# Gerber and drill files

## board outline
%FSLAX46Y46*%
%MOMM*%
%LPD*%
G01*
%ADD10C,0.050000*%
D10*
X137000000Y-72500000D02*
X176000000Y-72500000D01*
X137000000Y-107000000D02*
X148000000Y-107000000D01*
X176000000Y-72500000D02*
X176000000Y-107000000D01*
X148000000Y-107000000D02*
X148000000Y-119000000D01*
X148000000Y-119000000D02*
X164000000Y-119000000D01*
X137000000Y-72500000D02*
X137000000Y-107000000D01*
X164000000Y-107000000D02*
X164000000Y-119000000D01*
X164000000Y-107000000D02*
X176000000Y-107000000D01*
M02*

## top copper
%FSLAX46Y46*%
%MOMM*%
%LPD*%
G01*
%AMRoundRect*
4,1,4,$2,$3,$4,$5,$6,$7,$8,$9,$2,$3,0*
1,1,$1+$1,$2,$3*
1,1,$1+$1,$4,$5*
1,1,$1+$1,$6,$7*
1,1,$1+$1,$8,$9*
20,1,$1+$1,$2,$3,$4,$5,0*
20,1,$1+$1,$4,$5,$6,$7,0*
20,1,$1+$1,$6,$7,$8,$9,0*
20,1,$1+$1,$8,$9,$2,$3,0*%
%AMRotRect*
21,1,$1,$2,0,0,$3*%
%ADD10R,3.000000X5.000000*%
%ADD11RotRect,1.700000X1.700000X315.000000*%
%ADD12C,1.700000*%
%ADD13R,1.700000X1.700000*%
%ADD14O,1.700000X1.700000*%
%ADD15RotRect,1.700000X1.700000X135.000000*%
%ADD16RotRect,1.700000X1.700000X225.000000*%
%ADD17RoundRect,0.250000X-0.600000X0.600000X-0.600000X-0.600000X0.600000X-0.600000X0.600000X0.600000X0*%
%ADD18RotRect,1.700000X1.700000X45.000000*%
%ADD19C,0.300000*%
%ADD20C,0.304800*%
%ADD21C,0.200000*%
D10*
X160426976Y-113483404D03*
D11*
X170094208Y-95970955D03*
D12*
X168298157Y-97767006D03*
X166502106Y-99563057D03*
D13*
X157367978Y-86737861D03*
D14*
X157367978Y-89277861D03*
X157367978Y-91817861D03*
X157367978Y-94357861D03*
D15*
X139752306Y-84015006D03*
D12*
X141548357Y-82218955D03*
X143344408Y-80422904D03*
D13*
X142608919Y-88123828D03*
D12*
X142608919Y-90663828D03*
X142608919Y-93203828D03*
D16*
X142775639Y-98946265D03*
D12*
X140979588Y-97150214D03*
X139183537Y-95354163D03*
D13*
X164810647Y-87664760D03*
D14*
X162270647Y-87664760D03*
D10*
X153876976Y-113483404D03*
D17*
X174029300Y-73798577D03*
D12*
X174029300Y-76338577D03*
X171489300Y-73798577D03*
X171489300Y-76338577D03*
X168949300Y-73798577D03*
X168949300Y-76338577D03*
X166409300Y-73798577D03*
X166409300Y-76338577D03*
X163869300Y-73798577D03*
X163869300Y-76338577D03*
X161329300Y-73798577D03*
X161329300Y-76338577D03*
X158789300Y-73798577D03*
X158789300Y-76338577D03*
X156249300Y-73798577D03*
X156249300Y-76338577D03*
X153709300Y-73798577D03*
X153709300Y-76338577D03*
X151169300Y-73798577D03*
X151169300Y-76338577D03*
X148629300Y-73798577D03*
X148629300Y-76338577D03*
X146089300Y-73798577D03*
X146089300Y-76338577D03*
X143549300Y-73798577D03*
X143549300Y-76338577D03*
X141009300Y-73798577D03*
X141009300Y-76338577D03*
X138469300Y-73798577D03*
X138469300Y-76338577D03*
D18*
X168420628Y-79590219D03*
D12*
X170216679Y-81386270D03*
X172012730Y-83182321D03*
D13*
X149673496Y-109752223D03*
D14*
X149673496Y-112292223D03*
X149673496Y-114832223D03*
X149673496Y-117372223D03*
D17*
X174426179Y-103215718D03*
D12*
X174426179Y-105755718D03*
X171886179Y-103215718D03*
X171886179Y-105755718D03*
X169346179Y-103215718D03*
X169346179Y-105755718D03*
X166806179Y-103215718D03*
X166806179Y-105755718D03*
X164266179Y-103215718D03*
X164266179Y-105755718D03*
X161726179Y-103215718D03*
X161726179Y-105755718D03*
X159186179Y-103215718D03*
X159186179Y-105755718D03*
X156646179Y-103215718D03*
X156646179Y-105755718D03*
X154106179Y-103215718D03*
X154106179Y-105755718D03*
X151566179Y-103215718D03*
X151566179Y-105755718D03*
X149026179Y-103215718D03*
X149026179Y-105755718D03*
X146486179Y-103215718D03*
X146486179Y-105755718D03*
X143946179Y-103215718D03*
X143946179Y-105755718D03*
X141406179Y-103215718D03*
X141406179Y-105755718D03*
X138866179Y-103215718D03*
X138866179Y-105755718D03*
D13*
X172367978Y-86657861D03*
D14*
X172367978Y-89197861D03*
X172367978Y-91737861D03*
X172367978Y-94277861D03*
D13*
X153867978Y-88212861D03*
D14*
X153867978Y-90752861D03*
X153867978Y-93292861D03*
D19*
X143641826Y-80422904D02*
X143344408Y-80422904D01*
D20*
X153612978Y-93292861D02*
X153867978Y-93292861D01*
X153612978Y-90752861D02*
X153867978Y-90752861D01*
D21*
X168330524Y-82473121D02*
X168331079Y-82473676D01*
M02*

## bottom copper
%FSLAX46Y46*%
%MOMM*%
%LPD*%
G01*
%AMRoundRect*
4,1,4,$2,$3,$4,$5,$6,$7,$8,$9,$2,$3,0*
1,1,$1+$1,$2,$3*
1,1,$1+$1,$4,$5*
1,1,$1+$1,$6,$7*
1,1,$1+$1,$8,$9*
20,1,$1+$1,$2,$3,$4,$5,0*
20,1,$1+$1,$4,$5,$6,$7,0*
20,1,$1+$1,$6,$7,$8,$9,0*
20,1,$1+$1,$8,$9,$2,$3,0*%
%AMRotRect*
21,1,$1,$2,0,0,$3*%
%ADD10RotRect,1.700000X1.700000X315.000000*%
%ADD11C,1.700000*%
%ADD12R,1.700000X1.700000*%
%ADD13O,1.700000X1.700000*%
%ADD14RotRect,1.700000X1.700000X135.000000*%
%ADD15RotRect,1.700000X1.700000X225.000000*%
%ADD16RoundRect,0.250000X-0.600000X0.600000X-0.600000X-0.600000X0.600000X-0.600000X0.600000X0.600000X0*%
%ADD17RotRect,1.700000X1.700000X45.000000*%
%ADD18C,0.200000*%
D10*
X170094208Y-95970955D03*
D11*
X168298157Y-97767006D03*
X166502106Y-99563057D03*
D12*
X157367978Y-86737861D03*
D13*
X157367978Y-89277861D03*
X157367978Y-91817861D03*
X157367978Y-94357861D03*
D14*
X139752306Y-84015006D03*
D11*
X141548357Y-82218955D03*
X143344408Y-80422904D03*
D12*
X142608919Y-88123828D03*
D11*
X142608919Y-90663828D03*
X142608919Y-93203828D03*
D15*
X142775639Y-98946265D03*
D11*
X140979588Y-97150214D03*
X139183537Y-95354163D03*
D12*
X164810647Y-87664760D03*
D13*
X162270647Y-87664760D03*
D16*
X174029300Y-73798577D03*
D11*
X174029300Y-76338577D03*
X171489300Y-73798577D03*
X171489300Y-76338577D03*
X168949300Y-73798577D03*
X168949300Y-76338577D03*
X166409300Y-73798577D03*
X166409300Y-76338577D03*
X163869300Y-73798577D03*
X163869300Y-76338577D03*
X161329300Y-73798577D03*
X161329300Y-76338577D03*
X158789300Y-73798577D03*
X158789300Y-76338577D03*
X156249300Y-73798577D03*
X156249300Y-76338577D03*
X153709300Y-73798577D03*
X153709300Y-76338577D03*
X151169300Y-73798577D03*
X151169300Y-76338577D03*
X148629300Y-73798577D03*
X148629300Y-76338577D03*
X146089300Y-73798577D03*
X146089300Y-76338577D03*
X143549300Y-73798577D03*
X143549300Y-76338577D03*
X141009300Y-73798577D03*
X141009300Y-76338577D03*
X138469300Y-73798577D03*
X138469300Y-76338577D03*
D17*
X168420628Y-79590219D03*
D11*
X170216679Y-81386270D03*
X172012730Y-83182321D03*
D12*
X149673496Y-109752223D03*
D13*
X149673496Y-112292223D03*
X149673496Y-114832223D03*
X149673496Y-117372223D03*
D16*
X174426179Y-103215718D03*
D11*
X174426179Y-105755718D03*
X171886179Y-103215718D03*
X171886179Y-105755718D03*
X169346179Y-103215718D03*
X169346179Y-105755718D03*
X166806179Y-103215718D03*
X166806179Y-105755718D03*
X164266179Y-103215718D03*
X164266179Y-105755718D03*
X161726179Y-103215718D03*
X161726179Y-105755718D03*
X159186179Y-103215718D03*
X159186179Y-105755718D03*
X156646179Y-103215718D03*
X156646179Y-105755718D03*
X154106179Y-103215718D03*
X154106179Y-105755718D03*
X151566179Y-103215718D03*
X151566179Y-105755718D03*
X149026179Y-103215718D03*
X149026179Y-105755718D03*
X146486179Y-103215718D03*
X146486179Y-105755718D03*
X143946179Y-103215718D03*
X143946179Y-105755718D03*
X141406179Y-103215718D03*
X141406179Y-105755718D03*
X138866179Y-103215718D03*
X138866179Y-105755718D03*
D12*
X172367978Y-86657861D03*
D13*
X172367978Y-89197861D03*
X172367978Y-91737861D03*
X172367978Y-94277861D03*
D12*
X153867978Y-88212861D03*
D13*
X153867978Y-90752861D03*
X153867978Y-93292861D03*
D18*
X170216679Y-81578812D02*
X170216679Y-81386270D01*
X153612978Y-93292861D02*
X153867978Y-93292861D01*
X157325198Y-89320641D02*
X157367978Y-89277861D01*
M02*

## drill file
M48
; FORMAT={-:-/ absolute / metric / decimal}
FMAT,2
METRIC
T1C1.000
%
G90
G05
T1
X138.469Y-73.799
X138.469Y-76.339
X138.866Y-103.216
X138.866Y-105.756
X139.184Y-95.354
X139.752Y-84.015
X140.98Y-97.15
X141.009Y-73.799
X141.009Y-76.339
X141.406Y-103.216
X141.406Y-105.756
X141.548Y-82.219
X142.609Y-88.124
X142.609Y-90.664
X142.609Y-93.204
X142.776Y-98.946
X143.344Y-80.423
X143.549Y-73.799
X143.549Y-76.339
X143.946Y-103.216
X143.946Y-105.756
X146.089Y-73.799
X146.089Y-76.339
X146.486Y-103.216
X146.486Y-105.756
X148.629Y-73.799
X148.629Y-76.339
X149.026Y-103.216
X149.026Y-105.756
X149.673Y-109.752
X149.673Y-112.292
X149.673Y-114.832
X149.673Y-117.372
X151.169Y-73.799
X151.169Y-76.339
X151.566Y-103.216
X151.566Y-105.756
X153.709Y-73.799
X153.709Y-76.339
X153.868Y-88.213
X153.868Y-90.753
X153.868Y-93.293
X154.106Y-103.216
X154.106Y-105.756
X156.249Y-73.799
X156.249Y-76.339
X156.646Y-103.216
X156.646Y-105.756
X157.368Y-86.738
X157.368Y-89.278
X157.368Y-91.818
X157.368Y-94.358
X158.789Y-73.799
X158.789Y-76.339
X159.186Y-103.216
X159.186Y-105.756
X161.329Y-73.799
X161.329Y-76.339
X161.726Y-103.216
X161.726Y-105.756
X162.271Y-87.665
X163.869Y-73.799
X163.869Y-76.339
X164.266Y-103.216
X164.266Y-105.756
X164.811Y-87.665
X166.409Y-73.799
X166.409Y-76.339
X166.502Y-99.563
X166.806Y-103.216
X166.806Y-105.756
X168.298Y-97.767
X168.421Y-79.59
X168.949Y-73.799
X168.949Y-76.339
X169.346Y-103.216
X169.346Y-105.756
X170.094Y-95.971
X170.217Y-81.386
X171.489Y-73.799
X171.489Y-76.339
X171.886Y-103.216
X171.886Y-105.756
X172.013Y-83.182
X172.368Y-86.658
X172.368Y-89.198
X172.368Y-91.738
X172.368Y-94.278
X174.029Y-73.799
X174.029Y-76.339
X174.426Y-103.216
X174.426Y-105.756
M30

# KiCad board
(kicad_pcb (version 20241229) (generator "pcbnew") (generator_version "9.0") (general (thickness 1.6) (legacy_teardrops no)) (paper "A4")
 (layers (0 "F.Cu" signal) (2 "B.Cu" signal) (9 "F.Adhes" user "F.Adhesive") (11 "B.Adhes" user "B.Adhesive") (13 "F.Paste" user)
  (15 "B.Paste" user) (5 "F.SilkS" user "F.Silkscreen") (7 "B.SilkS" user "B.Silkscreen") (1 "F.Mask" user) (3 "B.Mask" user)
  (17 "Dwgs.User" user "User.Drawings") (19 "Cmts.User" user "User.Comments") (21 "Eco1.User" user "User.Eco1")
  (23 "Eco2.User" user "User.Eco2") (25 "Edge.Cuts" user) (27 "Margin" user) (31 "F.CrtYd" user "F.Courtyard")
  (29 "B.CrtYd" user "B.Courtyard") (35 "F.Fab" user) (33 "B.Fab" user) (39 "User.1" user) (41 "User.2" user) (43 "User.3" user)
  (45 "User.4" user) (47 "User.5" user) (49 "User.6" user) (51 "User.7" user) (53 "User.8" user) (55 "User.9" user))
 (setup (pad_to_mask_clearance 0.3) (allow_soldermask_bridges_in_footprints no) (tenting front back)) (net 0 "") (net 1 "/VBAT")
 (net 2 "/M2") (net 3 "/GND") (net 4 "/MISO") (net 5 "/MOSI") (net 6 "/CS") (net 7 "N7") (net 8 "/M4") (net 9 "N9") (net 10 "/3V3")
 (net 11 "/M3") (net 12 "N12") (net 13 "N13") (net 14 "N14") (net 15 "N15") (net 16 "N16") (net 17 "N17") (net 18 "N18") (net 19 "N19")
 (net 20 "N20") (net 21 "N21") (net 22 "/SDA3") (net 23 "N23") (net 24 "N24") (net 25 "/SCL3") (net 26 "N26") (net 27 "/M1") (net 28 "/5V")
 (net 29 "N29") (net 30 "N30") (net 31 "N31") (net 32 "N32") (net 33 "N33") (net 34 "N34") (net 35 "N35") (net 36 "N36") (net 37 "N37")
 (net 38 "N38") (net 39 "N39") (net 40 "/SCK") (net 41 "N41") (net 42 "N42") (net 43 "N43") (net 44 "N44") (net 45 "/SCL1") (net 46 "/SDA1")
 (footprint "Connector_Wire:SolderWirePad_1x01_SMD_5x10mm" (layer "F.Cu") (at 160.426976 107.783404)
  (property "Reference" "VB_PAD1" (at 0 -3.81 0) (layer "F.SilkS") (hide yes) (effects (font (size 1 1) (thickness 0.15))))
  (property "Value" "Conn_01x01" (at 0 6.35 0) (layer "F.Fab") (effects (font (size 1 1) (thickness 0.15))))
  (pad "1" smd rect (at 0 5.7) (size 3 5) (layers "F.Cu" "F.Mask" "F.Paste") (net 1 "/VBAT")))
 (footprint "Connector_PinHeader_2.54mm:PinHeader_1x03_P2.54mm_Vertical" (layer "F.Cu") (at 170.094208 95.970955 -45)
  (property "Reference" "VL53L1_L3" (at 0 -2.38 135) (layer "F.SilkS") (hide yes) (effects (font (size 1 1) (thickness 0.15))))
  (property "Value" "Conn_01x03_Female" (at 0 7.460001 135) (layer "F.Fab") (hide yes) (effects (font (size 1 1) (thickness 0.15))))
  (pad "1" thru_hole rect (at 0 0 315) (size 1.7 1.7) (drill 1) (layers "*.Cu" "*.Mask") (remove_unused_layers no) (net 1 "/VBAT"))
  (pad "2" thru_hole circle (at 0 2.54 315) (size 1.7 1.7) (drill 1) (layers "*.Cu" "*.Mask") (remove_unused_layers no) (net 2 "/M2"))
  (pad "3" thru_hole circle (at 0 5.079999 315) (size 1.7 1.7) (drill 1) (layers "*.Cu" "*.Mask") (remove_unused_layers no) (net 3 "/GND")))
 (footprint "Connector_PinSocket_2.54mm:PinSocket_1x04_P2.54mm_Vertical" (layer "F.Cu") (at 157.367978 86.737861)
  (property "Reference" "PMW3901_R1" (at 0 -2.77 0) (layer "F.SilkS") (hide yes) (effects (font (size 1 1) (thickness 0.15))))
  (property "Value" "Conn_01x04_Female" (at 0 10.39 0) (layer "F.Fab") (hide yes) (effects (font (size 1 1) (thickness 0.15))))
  (pad "1" thru_hole rect (at 0 0) (size 1.7 1.7) (drill 1) (layers "*.Cu" "*.Mask") (remove_unused_layers no) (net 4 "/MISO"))
  (pad "2" thru_hole oval (at 0 2.54) (size 1.7 1.7) (drill 1) (layers "*.Cu" "*.Mask") (remove_unused_layers no) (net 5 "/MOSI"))
  (pad "3" thru_hole oval (at 0 5.08) (size 1.7 1.7) (drill 1) (layers "*.Cu" "*.Mask") (remove_unused_layers no) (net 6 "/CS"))
  (pad "4" thru_hole oval (at 0 7.62) (size 1.7 1.7) (drill 1) (layers "*.Cu" "*.Mask") (remove_unused_layers no) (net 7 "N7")))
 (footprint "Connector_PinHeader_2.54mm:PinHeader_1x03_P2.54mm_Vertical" (layer "F.Cu") (at 139.752306 84.015006 135)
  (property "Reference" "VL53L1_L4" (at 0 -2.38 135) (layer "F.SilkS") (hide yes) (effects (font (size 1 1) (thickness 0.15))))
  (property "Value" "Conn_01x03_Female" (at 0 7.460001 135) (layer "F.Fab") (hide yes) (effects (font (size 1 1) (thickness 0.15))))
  (pad "1" thru_hole rect (at 0 0 135) (size 1.7 1.7) (drill 1) (layers "*.Cu" "*.Mask") (remove_unused_layers no) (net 1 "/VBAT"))
  (pad "2" thru_hole circle (at 0 2.54 135) (size 1.7 1.7) (drill 1) (layers "*.Cu" "*.Mask") (remove_unused_layers no) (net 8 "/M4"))
  (pad "3" thru_hole circle (at 0 5.079999 135) (size 1.7 1.7) (drill 1) (layers "*.Cu" "*.Mask") (remove_unused_layers no) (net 3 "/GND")))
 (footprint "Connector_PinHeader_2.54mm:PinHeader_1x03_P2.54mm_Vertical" (layer "F.Cu") (at 142.608919 88.123828)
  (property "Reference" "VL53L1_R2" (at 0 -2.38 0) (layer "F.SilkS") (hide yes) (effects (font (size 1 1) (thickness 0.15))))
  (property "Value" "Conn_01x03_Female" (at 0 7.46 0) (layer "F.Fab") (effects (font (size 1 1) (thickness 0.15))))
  (pad "1" thru_hole rect (at 0 0) (size 1.7 1.7) (drill 1) (layers "*.Cu" "*.Mask") (remove_unused_layers no) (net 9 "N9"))
  (pad "2" thru_hole circle (at 0 2.54) (size 1.7 1.7) (drill 1) (layers "*.Cu" "*.Mask") (remove_unused_layers no) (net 3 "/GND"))
  (pad "3" thru_hole circle (at 0 5.08) (size 1.7 1.7) (drill 1) (layers "*.Cu" "*.Mask") (remove_unused_layers no) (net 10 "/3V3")))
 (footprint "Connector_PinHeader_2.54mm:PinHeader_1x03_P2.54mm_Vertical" (layer "F.Cu") (at 142.775639 98.946265 -135)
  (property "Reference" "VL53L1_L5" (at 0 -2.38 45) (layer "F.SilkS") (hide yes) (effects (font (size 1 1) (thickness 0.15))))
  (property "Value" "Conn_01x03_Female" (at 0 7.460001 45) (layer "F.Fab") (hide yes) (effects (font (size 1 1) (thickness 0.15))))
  (pad "1" thru_hole rect (at 0 0 225) (size 1.7 1.7) (drill 1) (layers "*.Cu" "*.Mask") (remove_unused_layers no) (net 1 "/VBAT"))
  (pad "2" thru_hole circle (at 0 2.54 225) (size 1.7 1.7) (drill 1) (layers "*.Cu" "*.Mask") (remove_unused_layers no) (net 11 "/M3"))
  (pad "3" thru_hole circle (at 0 5.079999 225) (size 1.7 1.7) (drill 1) (layers "*.Cu" "*.Mask") (remove_unused_layers no) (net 3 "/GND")))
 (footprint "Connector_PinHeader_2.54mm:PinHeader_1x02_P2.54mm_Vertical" (layer "F.Cu") (at 164.810647 87.66476 -90)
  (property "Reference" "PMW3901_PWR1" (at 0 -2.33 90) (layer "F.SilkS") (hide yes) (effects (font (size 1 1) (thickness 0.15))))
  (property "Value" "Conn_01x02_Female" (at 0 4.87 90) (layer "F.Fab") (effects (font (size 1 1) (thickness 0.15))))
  (pad "1" thru_hole rect (at 0 0 270) (size 1.7 1.7) (drill 1) (layers "*.Cu" "*.Mask") (remove_unused_layers no) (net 3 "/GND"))
  (pad "2" thru_hole oval (at 0 2.54 270) (size 1.7 1.7) (drill 1) (layers "*.Cu" "*.Mask") (remove_unused_layers no) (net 10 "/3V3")))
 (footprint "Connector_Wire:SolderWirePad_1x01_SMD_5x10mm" (layer "F.Cu") (at 153.876976 107.783404)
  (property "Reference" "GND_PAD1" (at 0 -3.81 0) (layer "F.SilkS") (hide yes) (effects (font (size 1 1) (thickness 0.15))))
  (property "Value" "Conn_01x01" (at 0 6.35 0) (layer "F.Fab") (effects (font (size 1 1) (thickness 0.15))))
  (pad "1" smd rect (at 0 5.7) (size 3 5) (layers "F.Cu" "F.Mask" "F.Paste") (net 3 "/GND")))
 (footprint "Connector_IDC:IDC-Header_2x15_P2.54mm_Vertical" (layer "F.Cu") (at 174.0293 73.798577 -90)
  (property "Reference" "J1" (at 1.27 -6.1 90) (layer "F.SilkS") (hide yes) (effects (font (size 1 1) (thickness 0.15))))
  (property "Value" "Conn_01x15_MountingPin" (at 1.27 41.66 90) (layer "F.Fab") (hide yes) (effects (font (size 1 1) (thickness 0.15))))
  (pad "1" thru_hole roundrect (at 0 0 270) (size 1.7 1.7) (drill 1) (layers "*.Cu" "*.Mask") (remove_unused_layers no)
   (roundrect_rratio 0.147059) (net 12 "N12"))
  (pad "2" thru_hole circle (at 2.54 0 270) (size 1.7 1.7) (drill 1) (layers "*.Cu" "*.Mask") (remove_unused_layers no) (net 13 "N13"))
  (pad "3" thru_hole circle (at 0 2.54 270) (size 1.7 1.7) (drill 1) (layers "*.Cu" "*.Mask") (remove_unused_layers no) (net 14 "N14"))
  (pad "4" thru_hole circle (at 2.54 2.54 270) (size 1.7 1.7) (drill 1) (layers "*.Cu" "*.Mask") (remove_unused_layers no) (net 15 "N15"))
  (pad "5" thru_hole circle (at 0 5.08 270) (size 1.7 1.7) (drill 1) (layers "*.Cu" "*.Mask") (remove_unused_layers no) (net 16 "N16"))
  (pad "6" thru_hole circle (at 2.54 5.08 270) (size 1.7 1.7) (drill 1) (layers "*.Cu" "*.Mask") (remove_unused_layers no) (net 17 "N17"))
  (pad "7" thru_hole circle (at 0 7.62 270) (size 1.7 1.7) (drill 1) (layers "*.Cu" "*.Mask") (remove_unused_layers no) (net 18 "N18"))
  (pad "8" thru_hole circle (at 2.54 7.62 270) (size 1.7 1.7) (drill 1) (layers "*.Cu" "*.Mask") (remove_unused_layers no) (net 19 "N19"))
  (pad "9" thru_hole circle (at 0 10.16 270) (size 1.7 1.7) (drill 1) (layers "*.Cu" "*.Mask") (remove_unused_layers no) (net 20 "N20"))
  (pad "10" thru_hole circle (at 2.54 10.16 270) (size 1.7 1.7) (drill 1) (layers "*.Cu" "*.Mask") (remove_unused_layers no) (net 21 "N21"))
  (pad "11" thru_hole circle (at 0 12.7 270) (size 1.7 1.7) (drill 1) (layers "*.Cu" "*.Mask") (remove_unused_layers no) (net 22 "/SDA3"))
  (pad "12" thru_hole circle (at 2.54 12.7 270) (size 1.7 1.7) (drill 1) (layers "*.Cu" "*.Mask") (remove_unused_layers no) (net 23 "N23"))
  (pad "13" thru_hole circle (at 0 15.24 270) (size 1.7 1.7) (drill 1) (layers "*.Cu" "*.Mask") (remove_unused_layers no) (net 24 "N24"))
  (pad "14" thru_hole circle (at 2.54 15.24 270) (size 1.7 1.7) (drill 1) (layers "*.Cu" "*.Mask") (remove_unused_layers no)
   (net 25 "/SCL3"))
  (pad "15" thru_hole circle (at 0 17.78 270) (size 1.7 1.7) (drill 1) (layers "*.Cu" "*.Mask") (remove_unused_layers no) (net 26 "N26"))
  (pad "16" thru_hole circle (at 2.54 17.78 270) (size 1.7 1.7) (drill 1) (layers "*.Cu" "*.Mask") (remove_unused_layers no))
  (pad "17" thru_hole circle (at 0 20.32 270) (size 1.7 1.7) (drill 1) (layers "*.Cu" "*.Mask") (remove_unused_layers no))
  (pad "18" thru_hole circle (at 2.54 20.32 270) (size 1.7 1.7) (drill 1) (layers "*.Cu" "*.Mask") (remove_unused_layers no))
  (pad "19" thru_hole circle (at 0 22.86 270) (size 1.7 1.7) (drill 1) (layers "*.Cu" "*.Mask") (remove_unused_layers no))
  (pad "20" thru_hole circle (at 2.54 22.86 270) (size 1.7 1.7) (drill 1) (layers "*.Cu" "*.Mask") (remove_unused_layers no))
  (pad "21" thru_hole circle (at 0 25.4 270) (size 1.7 1.7) (drill 1) (layers "*.Cu" "*.Mask") (remove_unused_layers no))
  (pad "22" thru_hole circle (at 2.54 25.4 270) (size 1.7 1.7) (drill 1) (layers "*.Cu" "*.Mask") (remove_unused_layers no))
  (pad "23" thru_hole circle (at 0 27.94 270) (size 1.7 1.7) (drill 1) (layers "*.Cu" "*.Mask") (remove_unused_layers no))
  (pad "24" thru_hole circle (at 2.54 27.94 270) (size 1.7 1.7) (drill 1) (layers "*.Cu" "*.Mask") (remove_unused_layers no))
  (pad "25" thru_hole circle (at 0 30.48 270) (size 1.7 1.7) (drill 1) (layers "*.Cu" "*.Mask") (remove_unused_layers no))
  (pad "26" thru_hole circle (at 2.54 30.48 270) (size 1.7 1.7) (drill 1) (layers "*.Cu" "*.Mask") (remove_unused_layers no))
  (pad "27" thru_hole circle (at 0 33.02 270) (size 1.7 1.7) (drill 1) (layers "*.Cu" "*.Mask") (remove_unused_layers no))
  (pad "28" thru_hole circle (at 2.54 33.02 270) (size 1.7 1.7) (drill 1) (layers "*.Cu" "*.Mask") (remove_unused_layers no))
  (pad "29" thru_hole circle (at 0 35.56 270) (size 1.7 1.7) (drill 1) (layers "*.Cu" "*.Mask") (remove_unused_layers no))
  (pad "30" thru_hole circle (at 2.54 35.56 270) (size 1.7 1.7) (drill 1) (layers "*.Cu" "*.Mask") (remove_unused_layers no)))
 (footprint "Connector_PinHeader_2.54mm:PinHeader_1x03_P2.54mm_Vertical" (layer "F.Cu") (at 168.420628 79.590219 45)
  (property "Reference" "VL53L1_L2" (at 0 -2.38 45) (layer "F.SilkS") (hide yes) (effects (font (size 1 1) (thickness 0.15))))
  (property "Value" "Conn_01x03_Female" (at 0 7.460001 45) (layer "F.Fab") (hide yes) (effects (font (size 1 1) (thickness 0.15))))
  (pad "1" thru_hole rect (at 0 0 45) (size 1.7 1.7) (drill 1) (layers "*.Cu" "*.Mask") (remove_unused_layers no) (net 1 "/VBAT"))
  (pad "2" thru_hole circle (at 0 2.54 45) (size 1.7 1.7) (drill 1) (layers "*.Cu" "*.Mask") (remove_unused_layers no) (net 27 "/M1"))
  (pad "3" thru_hole circle (at 0 5.079999 45) (size 1.7 1.7) (drill 1) (layers "*.Cu" "*.Mask") (remove_unused_layers no) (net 3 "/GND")))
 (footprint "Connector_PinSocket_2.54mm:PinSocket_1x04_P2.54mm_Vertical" (layer "F.Cu") (at 149.673496 109.752223)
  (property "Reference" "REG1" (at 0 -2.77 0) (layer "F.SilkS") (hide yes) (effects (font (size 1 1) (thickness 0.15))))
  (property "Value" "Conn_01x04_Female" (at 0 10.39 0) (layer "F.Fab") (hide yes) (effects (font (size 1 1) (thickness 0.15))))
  (pad "1" thru_hole rect (at 0 0) (size 1.7 1.7) (drill 1) (layers "*.Cu" "*.Mask") (remove_unused_layers no) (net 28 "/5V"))
  (pad "2" thru_hole oval (at 0 2.54) (size 1.7 1.7) (drill 1) (layers "*.Cu" "*.Mask") (remove_unused_layers no) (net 3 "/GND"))
  (pad "3" thru_hole oval (at 0 5.08) (size 1.7 1.7) (drill 1) (layers "*.Cu" "*.Mask") (remove_unused_layers no) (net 1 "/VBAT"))
  (pad "4" thru_hole oval (at 0 7.62) (size 1.7 1.7) (drill 1) (layers "*.Cu" "*.Mask") (remove_unused_layers no) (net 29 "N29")))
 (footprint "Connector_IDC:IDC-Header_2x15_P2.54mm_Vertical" (layer "F.Cu") (at 174.426179 103.215718 -90)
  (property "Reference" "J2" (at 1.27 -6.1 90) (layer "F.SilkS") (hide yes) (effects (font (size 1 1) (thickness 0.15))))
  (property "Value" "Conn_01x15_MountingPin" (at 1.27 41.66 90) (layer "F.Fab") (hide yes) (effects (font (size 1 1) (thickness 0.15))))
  (pad "1" thru_hole roundrect (at 0 0 270) (size 1.7 1.7) (drill 1) (layers "*.Cu" "*.Mask") (remove_unused_layers no)
   (roundrect_rratio 0.147059) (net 10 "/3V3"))
  (pad "2" thru_hole circle (at 2.54 0 270) (size 1.7 1.7) (drill 1) (layers "*.Cu" "*.Mask") (remove_unused_layers no) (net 3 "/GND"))
  (pad "3" thru_hole circle (at 0 2.54 270) (size 1.7 1.7) (drill 1) (layers "*.Cu" "*.Mask") (remove_unused_layers no) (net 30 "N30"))
  (pad "4" thru_hole circle (at 2.54 2.54 270) (size 1.7 1.7) (drill 1) (layers "*.Cu" "*.Mask") (remove_unused_layers no) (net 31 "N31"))
  (pad "5" thru_hole circle (at 0 5.08 270) (size 1.7 1.7) (drill 1) (layers "*.Cu" "*.Mask") (remove_unused_layers no) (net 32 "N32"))
  (pad "6" thru_hole circle (at 2.54 5.08 270) (size 1.7 1.7) (drill 1) (layers "*.Cu" "*.Mask") (remove_unused_layers no) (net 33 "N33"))
  (pad "7" thru_hole circle (at 0 7.62 270) (size 1.7 1.7) (drill 1) (layers "*.Cu" "*.Mask") (remove_unused_layers no) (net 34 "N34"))
  (pad "8" thru_hole circle (at 2.54 7.62 270) (size 1.7 1.7) (drill 1) (layers "*.Cu" "*.Mask") (remove_unused_layers no) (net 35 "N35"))
  (pad "9" thru_hole circle (at 0 10.16 270) (size 1.7 1.7) (drill 1) (layers "*.Cu" "*.Mask") (remove_unused_layers no) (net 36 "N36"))
  (pad "10" thru_hole circle (at 2.54 10.16 270) (size 1.7 1.7) (drill 1) (layers "*.Cu" "*.Mask") (remove_unused_layers no) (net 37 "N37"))
  (pad "11" thru_hole circle (at 0 12.7 270) (size 1.7 1.7) (drill 1) (layers "*.Cu" "*.Mask") (remove_unused_layers no) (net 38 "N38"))
  (pad "12" thru_hole circle (at 2.54 12.7 270) (size 1.7 1.7) (drill 1) (layers "*.Cu" "*.Mask") (remove_unused_layers no) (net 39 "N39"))
  (pad "13" thru_hole circle (at 0 15.24 270) (size 1.7 1.7) (drill 1) (layers "*.Cu" "*.Mask") (remove_unused_layers no) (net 5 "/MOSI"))
  (pad "14" thru_hole circle (at 2.54 15.24 270) (size 1.7 1.7) (drill 1) (layers "*.Cu" "*.Mask") (remove_unused_layers no) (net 6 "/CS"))
  (pad "15" thru_hole circle (at 0 17.78 270) (size 1.7 1.7) (drill 1) (layers "*.Cu" "*.Mask") (remove_unused_layers no) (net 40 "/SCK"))
  (pad "16" thru_hole circle (at 2.54 17.78 270) (size 1.7 1.7) (drill 1) (layers "*.Cu" "*.Mask") (remove_unused_layers no) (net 4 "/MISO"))
  (pad "17" thru_hole circle (at 0 20.32 270) (size 1.7 1.7) (drill 1) (layers "*.Cu" "*.Mask") (remove_unused_layers no))
  (pad "18" thru_hole circle (at 2.54 20.32 270) (size 1.7 1.7) (drill 1) (layers "*.Cu" "*.Mask") (remove_unused_layers no))
  (pad "19" thru_hole circle (at 0 22.86 270) (size 1.7 1.7) (drill 1) (layers "*.Cu" "*.Mask") (remove_unused_layers no))
  (pad "20" thru_hole circle (at 2.54 22.86 270) (size 1.7 1.7) (drill 1) (layers "*.Cu" "*.Mask") (remove_unused_layers no))
  (pad "21" thru_hole circle (at 0 25.4 270) (size 1.7 1.7) (drill 1) (layers "*.Cu" "*.Mask") (remove_unused_layers no))
  (pad "22" thru_hole circle (at 2.54 25.4 270) (size 1.7 1.7) (drill 1) (layers "*.Cu" "*.Mask") (remove_unused_layers no))
  (pad "23" thru_hole circle (at 0 27.94 270) (size 1.7 1.7) (drill 1) (layers "*.Cu" "*.Mask") (remove_unused_layers no))
  (pad "24" thru_hole circle (at 2.54 27.94 270) (size 1.7 1.7) (drill 1) (layers "*.Cu" "*.Mask") (remove_unused_layers no))
  (pad "25" thru_hole circle (at 0 30.48 270) (size 1.7 1.7) (drill 1) (layers "*.Cu" "*.Mask") (remove_unused_layers no))
  (pad "26" thru_hole circle (at 2.54 30.48 270) (size 1.7 1.7) (drill 1) (layers "*.Cu" "*.Mask") (remove_unused_layers no))
  (pad "27" thru_hole circle (at 0 33.02 270) (size 1.7 1.7) (drill 1) (layers "*.Cu" "*.Mask") (remove_unused_layers no))
  (pad "28" thru_hole circle (at 2.54 33.02 270) (size 1.7 1.7) (drill 1) (layers "*.Cu" "*.Mask") (remove_unused_layers no))
  (pad "29" thru_hole circle (at 0 35.56 270) (size 1.7 1.7) (drill 1) (layers "*.Cu" "*.Mask") (remove_unused_layers no))
  (pad "30" thru_hole circle (at 2.54 35.56 270) (size 1.7 1.7) (drill 1) (layers "*.Cu" "*.Mask") (remove_unused_layers no)))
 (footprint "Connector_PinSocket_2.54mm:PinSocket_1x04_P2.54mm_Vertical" (layer "F.Cu") (at 172.367978 86.657861)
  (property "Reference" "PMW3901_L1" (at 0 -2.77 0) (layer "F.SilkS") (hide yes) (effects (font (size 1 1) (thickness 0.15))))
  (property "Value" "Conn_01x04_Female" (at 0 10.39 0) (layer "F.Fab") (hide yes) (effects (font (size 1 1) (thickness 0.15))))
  (pad "1" thru_hole rect (at 0 0) (size 1.7 1.7) (drill 1) (layers "*.Cu" "*.Mask") (remove_unused_layers no) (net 40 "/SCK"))
  (pad "2" thru_hole oval (at 0 2.54) (size 1.7 1.7) (drill 1) (layers "*.Cu" "*.Mask") (remove_unused_layers no) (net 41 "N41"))
  (pad "3" thru_hole oval (at 0 5.08) (size 1.7 1.7) (drill 1) (layers "*.Cu" "*.Mask") (remove_unused_layers no) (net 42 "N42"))
  (pad "4" thru_hole oval (at 0 7.62) (size 1.7 1.7) (drill 1) (layers "*.Cu" "*.Mask") (remove_unused_layers no) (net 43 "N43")))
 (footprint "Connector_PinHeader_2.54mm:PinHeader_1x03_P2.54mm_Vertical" (layer "F.Cu") (at 153.867978 88.212861)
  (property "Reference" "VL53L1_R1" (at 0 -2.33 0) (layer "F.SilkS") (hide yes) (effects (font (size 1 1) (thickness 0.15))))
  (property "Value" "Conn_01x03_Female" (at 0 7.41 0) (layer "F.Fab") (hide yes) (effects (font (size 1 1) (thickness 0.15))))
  (pad "1" thru_hole rect (at 0 0) (size 1.7 1.7) (drill 1) (layers "*.Cu" "*.Mask") (remove_unused_layers no) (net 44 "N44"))
  (pad "2" thru_hole oval (at 0 2.54) (size 1.7 1.7) (drill 1) (layers "*.Cu" "*.Mask") (remove_unused_layers no) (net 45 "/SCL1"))
  (pad "3" thru_hole oval (at 0 5.08) (size 1.7 1.7) (drill 1) (layers "*.Cu" "*.Mask") (remove_unused_layers no) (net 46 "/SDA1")))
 (gr_line (start 137 72.5) (end 176 72.5) (stroke (width 0.05) (type solid)) (layer "Edge.Cuts"))
 (gr_line (start 137 107) (end 148 107) (stroke (width 0.05) (type solid)) (layer "Edge.Cuts"))
 (gr_line (start 176 72.5) (end 176 107) (stroke (width 0.05) (type solid)) (layer "Edge.Cuts"))
 (gr_line (start 148 107) (end 148 119) (stroke (width 0.05) (type solid)) (layer "Edge.Cuts"))
 (gr_line (start 148 119) (end 164 119) (stroke (width 0.05) (type solid)) (layer "Edge.Cuts"))
 (gr_line (start 137 72.5) (end 137 107) (stroke (width 0.05) (type solid)) (layer "Edge.Cuts"))
 (gr_line (start 164 107) (end 164 119) (stroke (width 0.05) (type solid)) (layer "Edge.Cuts"))
 (gr_line (start 164 107) (end 176 107) (stroke (width 0.05) (type solid)) (layer "Edge.Cuts"))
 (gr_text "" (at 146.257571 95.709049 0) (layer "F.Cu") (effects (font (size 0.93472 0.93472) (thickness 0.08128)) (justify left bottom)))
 (segment (start 143.641826 80.422904) (end 143.344408 80.422904) (width 0.3) (layer "F.Cu") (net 3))
 (segment (start 170.216679 81.578812) (end 170.216679 81.38627) (width 0.2) (layer "B.Cu") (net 27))
 (segment (start 153.612978 93.292861) (end 153.867978 93.292861) (width 0.3048) (layer "F.Cu") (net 46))
 (segment (start 153.612978 93.292861) (end 153.867978 93.292861) (width 0.2) (layer "B.Cu") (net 46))
 (segment (start 153.612978 90.752861) (end 153.867978 90.752861) (width 0.3048) (layer "F.Cu") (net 45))
 (segment (start 168.330524 82.473121) (end 168.331079 82.473676) (width 0.2) (layer "F.Cu") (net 40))
 (segment (start 157.325198 89.320641) (end 157.367978 89.277861) (width 0.2) (layer "B.Cu") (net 5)))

